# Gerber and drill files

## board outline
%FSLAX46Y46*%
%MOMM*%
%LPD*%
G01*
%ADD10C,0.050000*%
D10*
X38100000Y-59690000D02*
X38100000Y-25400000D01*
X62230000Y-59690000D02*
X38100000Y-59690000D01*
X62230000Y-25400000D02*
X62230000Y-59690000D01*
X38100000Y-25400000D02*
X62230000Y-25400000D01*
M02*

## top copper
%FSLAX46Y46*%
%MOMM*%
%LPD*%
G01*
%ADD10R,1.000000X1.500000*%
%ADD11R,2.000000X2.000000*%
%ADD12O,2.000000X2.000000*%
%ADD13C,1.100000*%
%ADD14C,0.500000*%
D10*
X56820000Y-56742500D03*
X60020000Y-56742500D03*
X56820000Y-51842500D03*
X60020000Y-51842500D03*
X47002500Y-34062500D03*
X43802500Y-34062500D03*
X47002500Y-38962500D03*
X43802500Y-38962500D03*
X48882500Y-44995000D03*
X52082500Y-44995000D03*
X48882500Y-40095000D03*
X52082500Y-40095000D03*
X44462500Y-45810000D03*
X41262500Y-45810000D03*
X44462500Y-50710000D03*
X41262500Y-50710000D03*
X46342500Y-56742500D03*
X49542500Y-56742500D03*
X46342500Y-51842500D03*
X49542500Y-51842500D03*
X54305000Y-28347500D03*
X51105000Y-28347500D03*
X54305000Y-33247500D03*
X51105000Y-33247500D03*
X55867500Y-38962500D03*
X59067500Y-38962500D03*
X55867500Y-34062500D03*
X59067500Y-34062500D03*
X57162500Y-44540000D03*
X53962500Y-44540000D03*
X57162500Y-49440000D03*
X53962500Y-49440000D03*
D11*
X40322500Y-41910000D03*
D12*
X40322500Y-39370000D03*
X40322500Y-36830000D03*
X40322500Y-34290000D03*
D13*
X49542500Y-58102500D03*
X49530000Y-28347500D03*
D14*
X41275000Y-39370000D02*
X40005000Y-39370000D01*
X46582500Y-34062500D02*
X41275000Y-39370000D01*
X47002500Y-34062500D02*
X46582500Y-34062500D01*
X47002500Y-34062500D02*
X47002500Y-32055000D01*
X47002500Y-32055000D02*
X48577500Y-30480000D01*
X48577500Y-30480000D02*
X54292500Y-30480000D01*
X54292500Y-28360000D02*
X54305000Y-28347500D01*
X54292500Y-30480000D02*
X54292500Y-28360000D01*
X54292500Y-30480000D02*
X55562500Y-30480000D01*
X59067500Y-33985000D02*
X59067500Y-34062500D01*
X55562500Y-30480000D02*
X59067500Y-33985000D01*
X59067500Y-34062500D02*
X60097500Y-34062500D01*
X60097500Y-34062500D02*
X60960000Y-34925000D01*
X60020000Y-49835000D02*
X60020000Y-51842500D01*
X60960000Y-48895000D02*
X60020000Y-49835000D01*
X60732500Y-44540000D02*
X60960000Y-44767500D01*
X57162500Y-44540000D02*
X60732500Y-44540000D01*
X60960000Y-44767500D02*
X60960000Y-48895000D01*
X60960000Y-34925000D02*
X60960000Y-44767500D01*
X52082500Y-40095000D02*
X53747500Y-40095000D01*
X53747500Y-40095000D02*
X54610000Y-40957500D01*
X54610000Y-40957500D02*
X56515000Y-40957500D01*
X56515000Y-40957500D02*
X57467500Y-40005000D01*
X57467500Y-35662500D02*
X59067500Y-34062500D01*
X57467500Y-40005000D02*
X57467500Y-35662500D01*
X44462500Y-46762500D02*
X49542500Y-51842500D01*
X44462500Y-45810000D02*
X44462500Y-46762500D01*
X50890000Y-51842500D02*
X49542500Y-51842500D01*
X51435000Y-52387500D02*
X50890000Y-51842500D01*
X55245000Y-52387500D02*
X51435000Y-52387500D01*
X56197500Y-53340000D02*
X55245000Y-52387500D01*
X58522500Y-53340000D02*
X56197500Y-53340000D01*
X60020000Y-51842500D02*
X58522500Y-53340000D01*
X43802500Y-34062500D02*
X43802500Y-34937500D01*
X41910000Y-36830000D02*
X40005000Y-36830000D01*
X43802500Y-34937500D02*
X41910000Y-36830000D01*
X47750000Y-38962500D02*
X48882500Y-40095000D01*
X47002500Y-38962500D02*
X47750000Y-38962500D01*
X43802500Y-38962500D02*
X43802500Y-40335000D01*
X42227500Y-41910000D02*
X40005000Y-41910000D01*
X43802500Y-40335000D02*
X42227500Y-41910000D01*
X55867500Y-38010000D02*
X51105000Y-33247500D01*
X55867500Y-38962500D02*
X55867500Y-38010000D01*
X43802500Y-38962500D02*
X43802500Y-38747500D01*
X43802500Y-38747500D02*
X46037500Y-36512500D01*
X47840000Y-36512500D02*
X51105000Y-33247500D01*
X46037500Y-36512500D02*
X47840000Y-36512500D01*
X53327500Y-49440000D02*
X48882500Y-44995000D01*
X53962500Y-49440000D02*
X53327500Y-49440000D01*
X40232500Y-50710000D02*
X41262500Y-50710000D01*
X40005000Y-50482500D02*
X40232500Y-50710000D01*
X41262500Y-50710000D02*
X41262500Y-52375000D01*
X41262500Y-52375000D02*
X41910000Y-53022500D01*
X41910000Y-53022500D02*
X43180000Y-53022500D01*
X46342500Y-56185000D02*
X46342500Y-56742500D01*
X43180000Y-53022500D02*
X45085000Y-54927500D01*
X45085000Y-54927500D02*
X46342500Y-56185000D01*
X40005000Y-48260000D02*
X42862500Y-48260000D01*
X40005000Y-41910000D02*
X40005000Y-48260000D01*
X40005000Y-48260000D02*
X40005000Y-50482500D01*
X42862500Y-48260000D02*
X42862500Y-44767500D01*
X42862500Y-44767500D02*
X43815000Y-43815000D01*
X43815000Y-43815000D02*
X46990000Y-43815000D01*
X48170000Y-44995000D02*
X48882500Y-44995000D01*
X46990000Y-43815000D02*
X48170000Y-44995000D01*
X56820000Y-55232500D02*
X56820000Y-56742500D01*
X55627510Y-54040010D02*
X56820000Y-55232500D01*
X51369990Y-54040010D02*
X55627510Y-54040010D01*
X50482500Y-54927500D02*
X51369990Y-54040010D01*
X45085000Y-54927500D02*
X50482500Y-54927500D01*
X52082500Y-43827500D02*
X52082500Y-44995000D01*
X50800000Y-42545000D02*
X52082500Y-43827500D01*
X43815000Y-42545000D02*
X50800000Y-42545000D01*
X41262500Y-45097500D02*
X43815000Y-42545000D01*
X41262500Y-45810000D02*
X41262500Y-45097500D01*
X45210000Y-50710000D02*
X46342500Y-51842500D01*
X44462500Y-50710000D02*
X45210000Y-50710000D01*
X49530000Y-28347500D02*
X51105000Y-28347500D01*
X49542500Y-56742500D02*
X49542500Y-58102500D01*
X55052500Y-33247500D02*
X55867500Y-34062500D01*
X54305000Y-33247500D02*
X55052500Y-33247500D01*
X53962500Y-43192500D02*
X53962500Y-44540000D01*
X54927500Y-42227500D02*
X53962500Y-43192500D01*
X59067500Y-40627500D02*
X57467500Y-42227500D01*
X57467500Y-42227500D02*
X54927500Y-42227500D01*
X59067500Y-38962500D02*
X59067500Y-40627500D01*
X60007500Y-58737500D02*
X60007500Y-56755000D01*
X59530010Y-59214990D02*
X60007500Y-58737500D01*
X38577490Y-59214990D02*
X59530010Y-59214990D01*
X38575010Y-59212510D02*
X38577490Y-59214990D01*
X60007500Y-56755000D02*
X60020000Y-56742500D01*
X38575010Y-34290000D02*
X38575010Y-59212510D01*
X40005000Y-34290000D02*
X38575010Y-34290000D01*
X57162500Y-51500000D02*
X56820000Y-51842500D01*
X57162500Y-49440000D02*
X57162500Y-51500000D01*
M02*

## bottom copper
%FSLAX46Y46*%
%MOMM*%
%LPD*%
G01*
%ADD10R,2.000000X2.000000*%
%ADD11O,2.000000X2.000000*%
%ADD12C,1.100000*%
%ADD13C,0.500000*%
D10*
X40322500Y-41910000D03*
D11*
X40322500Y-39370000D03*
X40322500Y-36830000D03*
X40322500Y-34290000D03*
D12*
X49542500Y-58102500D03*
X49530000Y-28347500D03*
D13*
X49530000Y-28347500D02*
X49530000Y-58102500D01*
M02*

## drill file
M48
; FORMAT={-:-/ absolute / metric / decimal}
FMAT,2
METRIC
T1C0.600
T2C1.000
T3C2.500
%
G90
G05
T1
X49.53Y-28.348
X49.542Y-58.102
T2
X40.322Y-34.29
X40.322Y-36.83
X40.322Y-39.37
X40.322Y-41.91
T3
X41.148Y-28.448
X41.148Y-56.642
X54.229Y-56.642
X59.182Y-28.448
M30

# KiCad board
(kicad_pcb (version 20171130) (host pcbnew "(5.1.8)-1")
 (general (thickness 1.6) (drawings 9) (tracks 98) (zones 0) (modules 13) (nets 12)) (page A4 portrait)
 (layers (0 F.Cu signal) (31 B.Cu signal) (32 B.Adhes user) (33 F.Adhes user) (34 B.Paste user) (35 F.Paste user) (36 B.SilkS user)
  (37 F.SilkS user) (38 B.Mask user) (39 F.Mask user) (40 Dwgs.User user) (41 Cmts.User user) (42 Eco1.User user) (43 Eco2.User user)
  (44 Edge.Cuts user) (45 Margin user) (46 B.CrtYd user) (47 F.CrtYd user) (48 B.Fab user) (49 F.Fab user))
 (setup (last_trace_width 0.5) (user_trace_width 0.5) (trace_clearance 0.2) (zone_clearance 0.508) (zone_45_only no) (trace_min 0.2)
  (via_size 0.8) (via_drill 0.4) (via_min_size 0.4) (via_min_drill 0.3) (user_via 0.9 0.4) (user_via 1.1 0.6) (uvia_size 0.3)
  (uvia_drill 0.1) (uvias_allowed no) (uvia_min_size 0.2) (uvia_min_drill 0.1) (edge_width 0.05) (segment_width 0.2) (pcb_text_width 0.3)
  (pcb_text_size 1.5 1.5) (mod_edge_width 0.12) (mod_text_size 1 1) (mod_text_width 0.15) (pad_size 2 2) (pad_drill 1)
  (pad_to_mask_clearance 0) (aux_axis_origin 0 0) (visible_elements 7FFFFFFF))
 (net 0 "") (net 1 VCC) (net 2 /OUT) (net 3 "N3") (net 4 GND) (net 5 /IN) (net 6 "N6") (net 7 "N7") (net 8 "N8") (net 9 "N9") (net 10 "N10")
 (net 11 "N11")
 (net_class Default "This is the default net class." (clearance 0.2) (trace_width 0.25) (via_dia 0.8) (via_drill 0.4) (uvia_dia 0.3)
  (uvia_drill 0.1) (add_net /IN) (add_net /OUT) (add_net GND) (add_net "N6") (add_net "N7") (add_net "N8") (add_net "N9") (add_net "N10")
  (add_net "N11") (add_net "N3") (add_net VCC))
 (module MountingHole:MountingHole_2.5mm (layer F.Cu) (at 54.229 56.642)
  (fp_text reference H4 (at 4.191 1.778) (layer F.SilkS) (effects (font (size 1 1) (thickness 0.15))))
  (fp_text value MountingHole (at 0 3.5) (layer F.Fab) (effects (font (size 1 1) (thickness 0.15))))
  (pad 1 np_thru_hole circle (at 0 0) (size 2.5 2.5) (drill 2.5) (layers *.Cu *.Mask)))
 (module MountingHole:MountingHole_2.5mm (layer F.Cu) (at 41.148 56.642)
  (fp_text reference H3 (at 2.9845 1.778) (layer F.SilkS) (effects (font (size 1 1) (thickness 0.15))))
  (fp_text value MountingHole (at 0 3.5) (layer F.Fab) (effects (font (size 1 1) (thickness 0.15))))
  (pad 1 np_thru_hole circle (at 0 0) (size 2.5 2.5) (drill 2.5) (layers *.Cu *.Mask)))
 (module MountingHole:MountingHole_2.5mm (layer F.Cu) (at 59.182 28.448)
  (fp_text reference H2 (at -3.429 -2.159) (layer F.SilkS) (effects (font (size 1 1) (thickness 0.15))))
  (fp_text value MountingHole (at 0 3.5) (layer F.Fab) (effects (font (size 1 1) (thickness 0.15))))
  (pad 1 np_thru_hole circle (at 0 0) (size 2.5 2.5) (drill 2.5) (layers *.Cu *.Mask)))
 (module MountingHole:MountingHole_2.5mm (layer F.Cu) (at 41.148 28.448)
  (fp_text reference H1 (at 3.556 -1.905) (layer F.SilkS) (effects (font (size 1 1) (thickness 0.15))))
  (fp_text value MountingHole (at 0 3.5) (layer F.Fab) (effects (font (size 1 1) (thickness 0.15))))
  (pad 1 np_thru_hole circle (at 0 0) (size 2.5 2.5) (drill 2.5) (layers *.Cu *.Mask)))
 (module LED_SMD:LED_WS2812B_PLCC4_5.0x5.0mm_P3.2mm (layer F.Cu) (at 58.42 54.2925 90)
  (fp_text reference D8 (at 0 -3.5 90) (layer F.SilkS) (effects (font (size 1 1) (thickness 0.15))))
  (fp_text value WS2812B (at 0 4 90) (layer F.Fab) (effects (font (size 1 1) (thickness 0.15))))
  (pad 1 smd rect (at -2.45 -1.6 90) (size 1.5 1) (layers F.Cu F.Paste F.Mask) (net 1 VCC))
  (pad 2 smd rect (at -2.45 1.6 90) (size 1.5 1) (layers F.Cu F.Paste F.Mask) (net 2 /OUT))
  (pad 4 smd rect (at 2.45 -1.6 90) (size 1.5 1) (layers F.Cu F.Paste F.Mask) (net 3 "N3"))
  (pad 3 smd rect (at 2.45 1.6 90) (size 1.5 1) (layers F.Cu F.Paste F.Mask) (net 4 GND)))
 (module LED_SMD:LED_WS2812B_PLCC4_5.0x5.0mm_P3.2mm (layer F.Cu) (at 45.4025 36.5125 90)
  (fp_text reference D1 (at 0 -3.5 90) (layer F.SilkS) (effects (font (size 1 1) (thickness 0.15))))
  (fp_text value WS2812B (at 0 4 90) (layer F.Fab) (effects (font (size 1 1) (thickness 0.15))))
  (pad 3 smd rect (at 2.45 1.6 90) (size 1.5 1) (layers F.Cu F.Paste F.Mask) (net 4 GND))
  (pad 4 smd rect (at 2.45 -1.6 90) (size 1.5 1) (layers F.Cu F.Paste F.Mask) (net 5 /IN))
  (pad 2 smd rect (at -2.45 1.6 90) (size 1.5 1) (layers F.Cu F.Paste F.Mask) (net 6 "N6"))
  (pad 1 smd rect (at -2.45 -1.6 90) (size 1.5 1) (layers F.Cu F.Paste F.Mask) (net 1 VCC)))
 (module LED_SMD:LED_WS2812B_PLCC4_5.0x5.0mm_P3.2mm (layer F.Cu) (at 50.4825 42.545 90)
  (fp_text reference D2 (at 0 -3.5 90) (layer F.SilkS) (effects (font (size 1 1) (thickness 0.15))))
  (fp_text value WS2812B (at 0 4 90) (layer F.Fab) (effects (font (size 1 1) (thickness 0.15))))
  (pad 1 smd rect (at -2.45 -1.6 90) (size 1.5 1) (layers F.Cu F.Paste F.Mask) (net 1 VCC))
  (pad 2 smd rect (at -2.45 1.6 90) (size 1.5 1) (layers F.Cu F.Paste F.Mask) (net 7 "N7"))
  (pad 4 smd rect (at 2.45 -1.6 90) (size 1.5 1) (layers F.Cu F.Paste F.Mask) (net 6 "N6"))
  (pad 3 smd rect (at 2.45 1.6 90) (size 1.5 1) (layers F.Cu F.Paste F.Mask) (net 4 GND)))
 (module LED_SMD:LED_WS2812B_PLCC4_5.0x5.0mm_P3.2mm (layer F.Cu) (at 42.8625 48.26 90)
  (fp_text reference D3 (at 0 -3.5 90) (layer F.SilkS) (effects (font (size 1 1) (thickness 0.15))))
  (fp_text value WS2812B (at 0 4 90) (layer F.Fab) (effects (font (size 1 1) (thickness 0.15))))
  (pad 3 smd rect (at 2.45 1.6 90) (size 1.5 1) (layers F.Cu F.Paste F.Mask) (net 4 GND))
  (pad 4 smd rect (at 2.45 -1.6 90) (size 1.5 1) (layers F.Cu F.Paste F.Mask) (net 7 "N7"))
  (pad 2 smd rect (at -2.45 1.6 90) (size 1.5 1) (layers F.Cu F.Paste F.Mask) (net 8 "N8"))
  (pad 1 smd rect (at -2.45 -1.6 90) (size 1.5 1) (layers F.Cu F.Paste F.Mask) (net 1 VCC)))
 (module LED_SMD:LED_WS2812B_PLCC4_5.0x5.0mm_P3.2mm (layer F.Cu) (at 47.9425 54.2925 90)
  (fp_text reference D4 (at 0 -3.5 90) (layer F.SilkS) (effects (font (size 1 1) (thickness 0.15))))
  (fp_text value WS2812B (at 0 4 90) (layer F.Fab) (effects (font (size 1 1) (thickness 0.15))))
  (pad 1 smd rect (at -2.45 -1.6 90) (size 1.5 1) (layers F.Cu F.Paste F.Mask) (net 1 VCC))
  (pad 2 smd rect (at -2.45 1.6 90) (size 1.5 1) (layers F.Cu F.Paste F.Mask) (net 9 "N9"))
  (pad 4 smd rect (at 2.45 -1.6 90) (size 1.5 1) (layers F.Cu F.Paste F.Mask) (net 8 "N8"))
  (pad 3 smd rect (at 2.45 1.6 90) (size 1.5 1) (layers F.Cu F.Paste F.Mask) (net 4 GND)))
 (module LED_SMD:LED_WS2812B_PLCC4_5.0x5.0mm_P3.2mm (layer F.Cu) (at 52.705 30.7975 90)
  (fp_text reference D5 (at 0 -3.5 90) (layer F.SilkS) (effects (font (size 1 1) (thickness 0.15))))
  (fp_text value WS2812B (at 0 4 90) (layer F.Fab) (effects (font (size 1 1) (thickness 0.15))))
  (pad 3 smd rect (at 2.45 1.6 90) (size 1.5 1) (layers F.Cu F.Paste F.Mask) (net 4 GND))
  (pad 4 smd rect (at 2.45 -1.6 90) (size 1.5 1) (layers F.Cu F.Paste F.Mask) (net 9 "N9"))
  (pad 2 smd rect (at -2.45 1.6 90) (size 1.5 1) (layers F.Cu F.Paste F.Mask) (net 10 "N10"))
  (pad 1 smd rect (at -2.45 -1.6 90) (size 1.5 1) (layers F.Cu F.Paste F.Mask) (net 1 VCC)))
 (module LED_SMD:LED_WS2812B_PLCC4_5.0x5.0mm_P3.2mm (layer F.Cu) (at 57.4675 36.5125 90)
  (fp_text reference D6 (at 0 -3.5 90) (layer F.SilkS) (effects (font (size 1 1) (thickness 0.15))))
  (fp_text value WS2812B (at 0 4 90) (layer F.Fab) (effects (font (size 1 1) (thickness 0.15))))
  (pad 1 smd rect (at -2.45 -1.6 90) (size 1.5 1) (layers F.Cu F.Paste F.Mask) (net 1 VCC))
  (pad 2 smd rect (at -2.45 1.6 90) (size 1.5 1) (layers F.Cu F.Paste F.Mask) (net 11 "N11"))
  (pad 4 smd rect (at 2.45 -1.6 90) (size 1.5 1) (layers F.Cu F.Paste F.Mask) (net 10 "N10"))
  (pad 3 smd rect (at 2.45 1.6 90) (size 1.5 1) (layers F.Cu F.Paste F.Mask) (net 4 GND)))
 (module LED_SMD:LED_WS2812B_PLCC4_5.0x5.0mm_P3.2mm (layer F.Cu) (at 55.5625 46.99 90)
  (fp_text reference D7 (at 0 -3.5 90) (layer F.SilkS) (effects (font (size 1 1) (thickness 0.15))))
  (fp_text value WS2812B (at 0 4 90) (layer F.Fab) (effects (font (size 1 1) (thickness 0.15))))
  (pad 3 smd rect (at 2.45 1.6 90) (size 1.5 1) (layers F.Cu F.Paste F.Mask) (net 4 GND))
  (pad 4 smd rect (at 2.45 -1.6 90) (size 1.5 1) (layers F.Cu F.Paste F.Mask) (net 11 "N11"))
  (pad 2 smd rect (at -2.45 1.6 90) (size 1.5 1) (layers F.Cu F.Paste F.Mask) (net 3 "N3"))
  (pad 1 smd rect (at -2.45 -1.6 90) (size 1.5 1) (layers F.Cu F.Paste F.Mask) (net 1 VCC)))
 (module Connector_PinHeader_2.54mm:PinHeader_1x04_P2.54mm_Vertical (layer B.Cu) (at 40.3225 41.91)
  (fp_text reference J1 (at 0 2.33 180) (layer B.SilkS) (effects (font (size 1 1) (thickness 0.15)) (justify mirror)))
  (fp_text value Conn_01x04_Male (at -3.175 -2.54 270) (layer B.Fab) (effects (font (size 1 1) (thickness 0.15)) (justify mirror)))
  (pad 1 thru_hole rect (at 0 0) (size 2 2) (drill 1) (layers *.Cu *.Mask) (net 1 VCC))
  (pad 2 thru_hole oval (at 0 -2.54) (size 2 2) (drill 1) (layers *.Cu *.Mask) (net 4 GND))
  (pad 3 thru_hole oval (at 0 -5.08) (size 2 2) (drill 1) (layers *.Cu *.Mask) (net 5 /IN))
  (pad 4 thru_hole oval (at 0 -7.62) (size 2 2) (drill 1) (layers *.Cu *.Mask) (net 2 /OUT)))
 (gr_line (start 38.1 59.69) (end 38.1 25.4) (layer Edge.Cuts) (width 0.05))
 (gr_line (start 62.23 59.69) (end 38.1 59.69) (layer Edge.Cuts) (width 0.05))
 (gr_line (start 62.23 25.4) (end 62.23 59.69) (layer Edge.Cuts) (width 0.05))
 (gr_line (start 38.1 25.4) (end 62.23 25.4) (layer Edge.Cuts) (width 0.05))
 (segment (start 41.275 39.37) (end 40.005 39.37) (width 0.5) (layer F.Cu) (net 4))
 (segment (start 46.5825 34.0625) (end 41.275 39.37) (width 0.5) (layer F.Cu) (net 4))
 (segment (start 47.0025 34.0625) (end 46.5825 34.0625) (width 0.5) (layer F.Cu) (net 4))
 (segment (start 47.0025 34.0625) (end 47.0025 32.055) (width 0.5) (layer F.Cu) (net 4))
 (segment (start 47.0025 32.055) (end 48.5775 30.48) (width 0.5) (layer F.Cu) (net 4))
 (segment (start 48.5775 30.48) (end 54.2925 30.48) (width 0.5) (layer F.Cu) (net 4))
 (segment (start 54.2925 28.36) (end 54.305 28.3475) (width 0.5) (layer F.Cu) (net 4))
 (segment (start 54.2925 30.48) (end 54.2925 28.36) (width 0.5) (layer F.Cu) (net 4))
 (segment (start 54.2925 30.48) (end 55.5625 30.48) (width 0.5) (layer F.Cu) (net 4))
 (segment (start 59.0675 33.985) (end 59.0675 34.0625) (width 0.5) (layer F.Cu) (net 4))
 (segment (start 55.5625 30.48) (end 59.0675 33.985) (width 0.5) (layer F.Cu) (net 4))
 (segment (start 59.0675 34.0625) (end 60.0975 34.0625) (width 0.5) (layer F.Cu) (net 4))
 (segment (start 60.0975 34.0625) (end 60.96 34.925) (width 0.5) (layer F.Cu) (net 4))
 (segment (start 60.02 49.835) (end 60.02 51.8425) (width 0.5) (layer F.Cu) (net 4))
 (segment (start 60.96 48.895) (end 60.02 49.835) (width 0.5) (layer F.Cu) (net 4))
 (segment (start 60.7325 44.54) (end 60.96 44.7675) (width 0.5) (layer F.Cu) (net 4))
 (segment (start 57.1625 44.54) (end 60.7325 44.54) (width 0.5) (layer F.Cu) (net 4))
 (segment (start 60.96 44.7675) (end 60.96 48.895) (width 0.5) (layer F.Cu) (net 4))
 (segment (start 60.96 34.925) (end 60.96 44.7675) (width 0.5) (layer F.Cu) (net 4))
 (segment (start 52.0825 40.095) (end 53.7475 40.095) (width 0.5) (layer F.Cu) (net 4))
 (segment (start 53.7475 40.095) (end 54.61 40.9575) (width 0.5) (layer F.Cu) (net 4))
 (segment (start 54.61 40.9575) (end 56.515 40.9575) (width 0.5) (layer F.Cu) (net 4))
 (segment (start 56.515 40.9575) (end 57.4675 40.005) (width 0.5) (layer F.Cu) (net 4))
 (segment (start 57.4675 35.6625) (end 59.0675 34.0625) (width 0.5) (layer F.Cu) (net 4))
 (segment (start 57.4675 40.005) (end 57.4675 35.6625) (width 0.5) (layer F.Cu) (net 4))
 (segment (start 44.4625 46.7625) (end 49.5425 51.8425) (width 0.5) (layer F.Cu) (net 4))
 (segment (start 44.4625 45.81) (end 44.4625 46.7625) (width 0.5) (layer F.Cu) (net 4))
 (segment (start 50.89 51.8425) (end 49.5425 51.8425) (width 0.5) (layer F.Cu) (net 4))
 (segment (start 51.435 52.3875) (end 50.89 51.8425) (width 0.5) (layer F.Cu) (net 4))
 (segment (start 55.245 52.3875) (end 51.435 52.3875) (width 0.5) (layer F.Cu) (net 4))
 (segment (start 56.1975 53.34) (end 55.245 52.3875) (width 0.5) (layer F.Cu) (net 4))
 (segment (start 58.5225 53.34) (end 56.1975 53.34) (width 0.5) (layer F.Cu) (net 4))
 (segment (start 60.02 51.8425) (end 58.5225 53.34) (width 0.5) (layer F.Cu) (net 4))
 (segment (start 43.8025 34.0625) (end 43.8025 34.9375) (width 0.5) (layer F.Cu) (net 5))
 (segment (start 41.91 36.83) (end 40.005 36.83) (width 0.5) (layer F.Cu) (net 5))
 (segment (start 43.8025 34.9375) (end 41.91 36.83) (width 0.5) (layer F.Cu) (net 5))
 (segment (start 47.75 38.9625) (end 48.8825 40.095) (width 0.5) (layer F.Cu) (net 6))
 (segment (start 47.0025 38.9625) (end 47.75 38.9625) (width 0.5) (layer F.Cu) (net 6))
 (segment (start 43.8025 38.9625) (end 43.8025 40.335) (width 0.5) (layer F.Cu) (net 1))
 (segment (start 42.2275 41.91) (end 40.005 41.91) (width 0.5) (layer F.Cu) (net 1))
 (segment (start 43.8025 40.335) (end 42.2275 41.91) (width 0.5) (layer F.Cu) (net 1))
 (segment (start 55.8675 38.01) (end 51.105 33.2475) (width 0.5) (layer F.Cu) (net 1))
 (segment (start 55.8675 38.9625) (end 55.8675 38.01) (width 0.5) (layer F.Cu) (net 1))
 (segment (start 43.8025 38.9625) (end 43.8025 38.7475) (width 0.5) (layer F.Cu) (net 1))
 (segment (start 43.8025 38.7475) (end 46.0375 36.5125) (width 0.5) (layer F.Cu) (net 1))
 (segment (start 47.84 36.5125) (end 51.105 33.2475) (width 0.5) (layer F.Cu) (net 1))
 (segment (start 46.0375 36.5125) (end 47.84 36.5125) (width 0.5) (layer F.Cu) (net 1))
 (segment (start 53.3275 49.44) (end 48.8825 44.995) (width 0.5) (layer F.Cu) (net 1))
 (segment (start 53.9625 49.44) (end 53.3275 49.44) (width 0.5) (layer F.Cu) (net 1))
 (segment (start 40.2325 50.71) (end 41.2625 50.71) (width 0.5) (layer F.Cu) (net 1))
 (segment (start 40.005 50.4825) (end 40.2325 50.71) (width 0.5) (layer F.Cu) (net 1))
 (segment (start 41.2625 50.71) (end 41.2625 52.375) (width 0.5) (layer F.Cu) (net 1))
 (segment (start 41.2625 52.375) (end 41.91 53.0225) (width 0.5) (layer F.Cu) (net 1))
 (segment (start 41.91 53.0225) (end 43.18 53.0225) (width 0.5) (layer F.Cu) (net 1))
 (segment (start 46.3425 56.185) (end 46.3425 56.7425) (width 0.5) (layer F.Cu) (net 1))
 (segment (start 43.18 53.0225) (end 45.085 54.9275) (width 0.5) (layer F.Cu) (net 1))
 (segment (start 45.085 54.9275) (end 46.3425 56.185) (width 0.5) (layer F.Cu) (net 1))
 (segment (start 40.005 48.26) (end 42.8625 48.26) (width 0.5) (layer F.Cu) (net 1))
 (segment (start 40.005 41.91) (end 40.005 48.26) (width 0.5) (layer F.Cu) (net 1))
 (segment (start 40.005 48.26) (end 40.005 50.4825) (width 0.5) (layer F.Cu) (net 1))
 (segment (start 42.8625 48.26) (end 42.8625 44.7675) (width 0.5) (layer F.Cu) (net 1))
 (segment (start 42.8625 44.7675) (end 43.815 43.815) (width 0.5) (layer F.Cu) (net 1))
 (segment (start 43.815 43.815) (end 46.99 43.815) (width 0.5) (layer F.Cu) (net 1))
 (segment (start 48.17 44.995) (end 48.8825 44.995) (width 0.5) (layer F.Cu) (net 1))
 (segment (start 46.99 43.815) (end 48.17 44.995) (width 0.5) (layer F.Cu) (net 1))
 (segment (start 56.82 55.2325) (end 56.82 56.7425) (width 0.5) (layer F.Cu) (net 1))
 (segment (start 55.62751 54.04001) (end 56.82 55.2325) (width 0.5) (layer F.Cu) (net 1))
 (segment (start 51.36999 54.04001) (end 55.62751 54.04001) (width 0.5) (layer F.Cu) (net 1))
 (segment (start 50.4825 54.9275) (end 51.36999 54.04001) (width 0.5) (layer F.Cu) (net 1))
 (segment (start 45.085 54.9275) (end 50.4825 54.9275) (width 0.5) (layer F.Cu) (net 1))
 (segment (start 52.0825 43.8275) (end 52.0825 44.995) (width 0.5) (layer F.Cu) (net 7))
 (segment (start 50.8 42.545) (end 52.0825 43.8275) (width 0.5) (layer F.Cu) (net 7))
 (segment (start 43.815 42.545) (end 50.8 42.545) (width 0.5) (layer F.Cu) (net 7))
 (segment (start 41.2625 45.0975) (end 43.815 42.545) (width 0.5) (layer F.Cu) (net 7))
 (segment (start 41.2625 45.81) (end 41.2625 45.0975) (width 0.5) (layer F.Cu) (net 7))
 (segment (start 45.21 50.71) (end 46.3425 51.8425) (width 0.5) (layer F.Cu) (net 8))
 (segment (start 44.4625 50.71) (end 45.21 50.71) (width 0.5) (layer F.Cu) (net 8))
 (via (at 49.5425 58.1025) (size 1.1) (drill 0.6) (layers F.Cu B.Cu) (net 9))
 (via (at 49.53 28.3475) (size 1.1) (drill 0.6) (layers F.Cu B.Cu) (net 9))
 (segment (start 49.53 28.3475) (end 51.105 28.3475) (width 0.5) (layer F.Cu) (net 9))
 (segment (start 49.53 28.3475) (end 49.53 58.1025) (width 0.5) (layer B.Cu) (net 9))
 (segment (start 49.5425 56.7425) (end 49.5425 58.1025) (width 0.5) (layer F.Cu) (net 9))
 (segment (start 55.0525 33.2475) (end 55.8675 34.0625) (width 0.5) (layer F.Cu) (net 10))
 (segment (start 54.305 33.2475) (end 55.0525 33.2475) (width 0.5) (layer F.Cu) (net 10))
 (segment (start 53.9625 43.1925) (end 53.9625 44.54) (width 0.5) (layer F.Cu) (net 11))
 (segment (start 54.9275 42.2275) (end 53.9625 43.1925) (width 0.5) (layer F.Cu) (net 11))
 (segment (start 59.0675 40.6275) (end 57.4675 42.2275) (width 0.5) (layer F.Cu) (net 11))
 (segment (start 57.4675 42.2275) (end 54.9275 42.2275) (width 0.5) (layer F.Cu) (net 11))
 (segment (start 59.0675 38.9625) (end 59.0675 40.6275) (width 0.5) (layer F.Cu) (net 11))
 (segment (start 60.0075 58.7375) (end 60.0075 56.755) (width 0.5) (layer F.Cu) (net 2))
 (segment (start 59.53001 59.21499) (end 60.0075 58.7375) (width 0.5) (layer F.Cu) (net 2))
 (segment (start 38.57749 59.21499) (end 59.53001 59.21499) (width 0.5) (layer F.Cu) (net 2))
 (segment (start 38.57501 59.21251) (end 38.57749 59.21499) (width 0.5) (layer F.Cu) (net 2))
 (segment (start 60.0075 56.755) (end 60.02 56.7425) (width 0.5) (layer F.Cu) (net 2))
 (segment (start 38.57501 34.29) (end 38.57501 59.21251) (width 0.5) (layer F.Cu) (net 2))
 (segment (start 40.005 34.29) (end 38.57501 34.29) (width 0.5) (layer F.Cu) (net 2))
 (segment (start 57.1625 51.5) (end 56.82 51.8425) (width 0.5) (layer F.Cu) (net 3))
 (segment (start 57.1625 49.44) (end 57.1625 51.5) (width 0.5) (layer F.Cu) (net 3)))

